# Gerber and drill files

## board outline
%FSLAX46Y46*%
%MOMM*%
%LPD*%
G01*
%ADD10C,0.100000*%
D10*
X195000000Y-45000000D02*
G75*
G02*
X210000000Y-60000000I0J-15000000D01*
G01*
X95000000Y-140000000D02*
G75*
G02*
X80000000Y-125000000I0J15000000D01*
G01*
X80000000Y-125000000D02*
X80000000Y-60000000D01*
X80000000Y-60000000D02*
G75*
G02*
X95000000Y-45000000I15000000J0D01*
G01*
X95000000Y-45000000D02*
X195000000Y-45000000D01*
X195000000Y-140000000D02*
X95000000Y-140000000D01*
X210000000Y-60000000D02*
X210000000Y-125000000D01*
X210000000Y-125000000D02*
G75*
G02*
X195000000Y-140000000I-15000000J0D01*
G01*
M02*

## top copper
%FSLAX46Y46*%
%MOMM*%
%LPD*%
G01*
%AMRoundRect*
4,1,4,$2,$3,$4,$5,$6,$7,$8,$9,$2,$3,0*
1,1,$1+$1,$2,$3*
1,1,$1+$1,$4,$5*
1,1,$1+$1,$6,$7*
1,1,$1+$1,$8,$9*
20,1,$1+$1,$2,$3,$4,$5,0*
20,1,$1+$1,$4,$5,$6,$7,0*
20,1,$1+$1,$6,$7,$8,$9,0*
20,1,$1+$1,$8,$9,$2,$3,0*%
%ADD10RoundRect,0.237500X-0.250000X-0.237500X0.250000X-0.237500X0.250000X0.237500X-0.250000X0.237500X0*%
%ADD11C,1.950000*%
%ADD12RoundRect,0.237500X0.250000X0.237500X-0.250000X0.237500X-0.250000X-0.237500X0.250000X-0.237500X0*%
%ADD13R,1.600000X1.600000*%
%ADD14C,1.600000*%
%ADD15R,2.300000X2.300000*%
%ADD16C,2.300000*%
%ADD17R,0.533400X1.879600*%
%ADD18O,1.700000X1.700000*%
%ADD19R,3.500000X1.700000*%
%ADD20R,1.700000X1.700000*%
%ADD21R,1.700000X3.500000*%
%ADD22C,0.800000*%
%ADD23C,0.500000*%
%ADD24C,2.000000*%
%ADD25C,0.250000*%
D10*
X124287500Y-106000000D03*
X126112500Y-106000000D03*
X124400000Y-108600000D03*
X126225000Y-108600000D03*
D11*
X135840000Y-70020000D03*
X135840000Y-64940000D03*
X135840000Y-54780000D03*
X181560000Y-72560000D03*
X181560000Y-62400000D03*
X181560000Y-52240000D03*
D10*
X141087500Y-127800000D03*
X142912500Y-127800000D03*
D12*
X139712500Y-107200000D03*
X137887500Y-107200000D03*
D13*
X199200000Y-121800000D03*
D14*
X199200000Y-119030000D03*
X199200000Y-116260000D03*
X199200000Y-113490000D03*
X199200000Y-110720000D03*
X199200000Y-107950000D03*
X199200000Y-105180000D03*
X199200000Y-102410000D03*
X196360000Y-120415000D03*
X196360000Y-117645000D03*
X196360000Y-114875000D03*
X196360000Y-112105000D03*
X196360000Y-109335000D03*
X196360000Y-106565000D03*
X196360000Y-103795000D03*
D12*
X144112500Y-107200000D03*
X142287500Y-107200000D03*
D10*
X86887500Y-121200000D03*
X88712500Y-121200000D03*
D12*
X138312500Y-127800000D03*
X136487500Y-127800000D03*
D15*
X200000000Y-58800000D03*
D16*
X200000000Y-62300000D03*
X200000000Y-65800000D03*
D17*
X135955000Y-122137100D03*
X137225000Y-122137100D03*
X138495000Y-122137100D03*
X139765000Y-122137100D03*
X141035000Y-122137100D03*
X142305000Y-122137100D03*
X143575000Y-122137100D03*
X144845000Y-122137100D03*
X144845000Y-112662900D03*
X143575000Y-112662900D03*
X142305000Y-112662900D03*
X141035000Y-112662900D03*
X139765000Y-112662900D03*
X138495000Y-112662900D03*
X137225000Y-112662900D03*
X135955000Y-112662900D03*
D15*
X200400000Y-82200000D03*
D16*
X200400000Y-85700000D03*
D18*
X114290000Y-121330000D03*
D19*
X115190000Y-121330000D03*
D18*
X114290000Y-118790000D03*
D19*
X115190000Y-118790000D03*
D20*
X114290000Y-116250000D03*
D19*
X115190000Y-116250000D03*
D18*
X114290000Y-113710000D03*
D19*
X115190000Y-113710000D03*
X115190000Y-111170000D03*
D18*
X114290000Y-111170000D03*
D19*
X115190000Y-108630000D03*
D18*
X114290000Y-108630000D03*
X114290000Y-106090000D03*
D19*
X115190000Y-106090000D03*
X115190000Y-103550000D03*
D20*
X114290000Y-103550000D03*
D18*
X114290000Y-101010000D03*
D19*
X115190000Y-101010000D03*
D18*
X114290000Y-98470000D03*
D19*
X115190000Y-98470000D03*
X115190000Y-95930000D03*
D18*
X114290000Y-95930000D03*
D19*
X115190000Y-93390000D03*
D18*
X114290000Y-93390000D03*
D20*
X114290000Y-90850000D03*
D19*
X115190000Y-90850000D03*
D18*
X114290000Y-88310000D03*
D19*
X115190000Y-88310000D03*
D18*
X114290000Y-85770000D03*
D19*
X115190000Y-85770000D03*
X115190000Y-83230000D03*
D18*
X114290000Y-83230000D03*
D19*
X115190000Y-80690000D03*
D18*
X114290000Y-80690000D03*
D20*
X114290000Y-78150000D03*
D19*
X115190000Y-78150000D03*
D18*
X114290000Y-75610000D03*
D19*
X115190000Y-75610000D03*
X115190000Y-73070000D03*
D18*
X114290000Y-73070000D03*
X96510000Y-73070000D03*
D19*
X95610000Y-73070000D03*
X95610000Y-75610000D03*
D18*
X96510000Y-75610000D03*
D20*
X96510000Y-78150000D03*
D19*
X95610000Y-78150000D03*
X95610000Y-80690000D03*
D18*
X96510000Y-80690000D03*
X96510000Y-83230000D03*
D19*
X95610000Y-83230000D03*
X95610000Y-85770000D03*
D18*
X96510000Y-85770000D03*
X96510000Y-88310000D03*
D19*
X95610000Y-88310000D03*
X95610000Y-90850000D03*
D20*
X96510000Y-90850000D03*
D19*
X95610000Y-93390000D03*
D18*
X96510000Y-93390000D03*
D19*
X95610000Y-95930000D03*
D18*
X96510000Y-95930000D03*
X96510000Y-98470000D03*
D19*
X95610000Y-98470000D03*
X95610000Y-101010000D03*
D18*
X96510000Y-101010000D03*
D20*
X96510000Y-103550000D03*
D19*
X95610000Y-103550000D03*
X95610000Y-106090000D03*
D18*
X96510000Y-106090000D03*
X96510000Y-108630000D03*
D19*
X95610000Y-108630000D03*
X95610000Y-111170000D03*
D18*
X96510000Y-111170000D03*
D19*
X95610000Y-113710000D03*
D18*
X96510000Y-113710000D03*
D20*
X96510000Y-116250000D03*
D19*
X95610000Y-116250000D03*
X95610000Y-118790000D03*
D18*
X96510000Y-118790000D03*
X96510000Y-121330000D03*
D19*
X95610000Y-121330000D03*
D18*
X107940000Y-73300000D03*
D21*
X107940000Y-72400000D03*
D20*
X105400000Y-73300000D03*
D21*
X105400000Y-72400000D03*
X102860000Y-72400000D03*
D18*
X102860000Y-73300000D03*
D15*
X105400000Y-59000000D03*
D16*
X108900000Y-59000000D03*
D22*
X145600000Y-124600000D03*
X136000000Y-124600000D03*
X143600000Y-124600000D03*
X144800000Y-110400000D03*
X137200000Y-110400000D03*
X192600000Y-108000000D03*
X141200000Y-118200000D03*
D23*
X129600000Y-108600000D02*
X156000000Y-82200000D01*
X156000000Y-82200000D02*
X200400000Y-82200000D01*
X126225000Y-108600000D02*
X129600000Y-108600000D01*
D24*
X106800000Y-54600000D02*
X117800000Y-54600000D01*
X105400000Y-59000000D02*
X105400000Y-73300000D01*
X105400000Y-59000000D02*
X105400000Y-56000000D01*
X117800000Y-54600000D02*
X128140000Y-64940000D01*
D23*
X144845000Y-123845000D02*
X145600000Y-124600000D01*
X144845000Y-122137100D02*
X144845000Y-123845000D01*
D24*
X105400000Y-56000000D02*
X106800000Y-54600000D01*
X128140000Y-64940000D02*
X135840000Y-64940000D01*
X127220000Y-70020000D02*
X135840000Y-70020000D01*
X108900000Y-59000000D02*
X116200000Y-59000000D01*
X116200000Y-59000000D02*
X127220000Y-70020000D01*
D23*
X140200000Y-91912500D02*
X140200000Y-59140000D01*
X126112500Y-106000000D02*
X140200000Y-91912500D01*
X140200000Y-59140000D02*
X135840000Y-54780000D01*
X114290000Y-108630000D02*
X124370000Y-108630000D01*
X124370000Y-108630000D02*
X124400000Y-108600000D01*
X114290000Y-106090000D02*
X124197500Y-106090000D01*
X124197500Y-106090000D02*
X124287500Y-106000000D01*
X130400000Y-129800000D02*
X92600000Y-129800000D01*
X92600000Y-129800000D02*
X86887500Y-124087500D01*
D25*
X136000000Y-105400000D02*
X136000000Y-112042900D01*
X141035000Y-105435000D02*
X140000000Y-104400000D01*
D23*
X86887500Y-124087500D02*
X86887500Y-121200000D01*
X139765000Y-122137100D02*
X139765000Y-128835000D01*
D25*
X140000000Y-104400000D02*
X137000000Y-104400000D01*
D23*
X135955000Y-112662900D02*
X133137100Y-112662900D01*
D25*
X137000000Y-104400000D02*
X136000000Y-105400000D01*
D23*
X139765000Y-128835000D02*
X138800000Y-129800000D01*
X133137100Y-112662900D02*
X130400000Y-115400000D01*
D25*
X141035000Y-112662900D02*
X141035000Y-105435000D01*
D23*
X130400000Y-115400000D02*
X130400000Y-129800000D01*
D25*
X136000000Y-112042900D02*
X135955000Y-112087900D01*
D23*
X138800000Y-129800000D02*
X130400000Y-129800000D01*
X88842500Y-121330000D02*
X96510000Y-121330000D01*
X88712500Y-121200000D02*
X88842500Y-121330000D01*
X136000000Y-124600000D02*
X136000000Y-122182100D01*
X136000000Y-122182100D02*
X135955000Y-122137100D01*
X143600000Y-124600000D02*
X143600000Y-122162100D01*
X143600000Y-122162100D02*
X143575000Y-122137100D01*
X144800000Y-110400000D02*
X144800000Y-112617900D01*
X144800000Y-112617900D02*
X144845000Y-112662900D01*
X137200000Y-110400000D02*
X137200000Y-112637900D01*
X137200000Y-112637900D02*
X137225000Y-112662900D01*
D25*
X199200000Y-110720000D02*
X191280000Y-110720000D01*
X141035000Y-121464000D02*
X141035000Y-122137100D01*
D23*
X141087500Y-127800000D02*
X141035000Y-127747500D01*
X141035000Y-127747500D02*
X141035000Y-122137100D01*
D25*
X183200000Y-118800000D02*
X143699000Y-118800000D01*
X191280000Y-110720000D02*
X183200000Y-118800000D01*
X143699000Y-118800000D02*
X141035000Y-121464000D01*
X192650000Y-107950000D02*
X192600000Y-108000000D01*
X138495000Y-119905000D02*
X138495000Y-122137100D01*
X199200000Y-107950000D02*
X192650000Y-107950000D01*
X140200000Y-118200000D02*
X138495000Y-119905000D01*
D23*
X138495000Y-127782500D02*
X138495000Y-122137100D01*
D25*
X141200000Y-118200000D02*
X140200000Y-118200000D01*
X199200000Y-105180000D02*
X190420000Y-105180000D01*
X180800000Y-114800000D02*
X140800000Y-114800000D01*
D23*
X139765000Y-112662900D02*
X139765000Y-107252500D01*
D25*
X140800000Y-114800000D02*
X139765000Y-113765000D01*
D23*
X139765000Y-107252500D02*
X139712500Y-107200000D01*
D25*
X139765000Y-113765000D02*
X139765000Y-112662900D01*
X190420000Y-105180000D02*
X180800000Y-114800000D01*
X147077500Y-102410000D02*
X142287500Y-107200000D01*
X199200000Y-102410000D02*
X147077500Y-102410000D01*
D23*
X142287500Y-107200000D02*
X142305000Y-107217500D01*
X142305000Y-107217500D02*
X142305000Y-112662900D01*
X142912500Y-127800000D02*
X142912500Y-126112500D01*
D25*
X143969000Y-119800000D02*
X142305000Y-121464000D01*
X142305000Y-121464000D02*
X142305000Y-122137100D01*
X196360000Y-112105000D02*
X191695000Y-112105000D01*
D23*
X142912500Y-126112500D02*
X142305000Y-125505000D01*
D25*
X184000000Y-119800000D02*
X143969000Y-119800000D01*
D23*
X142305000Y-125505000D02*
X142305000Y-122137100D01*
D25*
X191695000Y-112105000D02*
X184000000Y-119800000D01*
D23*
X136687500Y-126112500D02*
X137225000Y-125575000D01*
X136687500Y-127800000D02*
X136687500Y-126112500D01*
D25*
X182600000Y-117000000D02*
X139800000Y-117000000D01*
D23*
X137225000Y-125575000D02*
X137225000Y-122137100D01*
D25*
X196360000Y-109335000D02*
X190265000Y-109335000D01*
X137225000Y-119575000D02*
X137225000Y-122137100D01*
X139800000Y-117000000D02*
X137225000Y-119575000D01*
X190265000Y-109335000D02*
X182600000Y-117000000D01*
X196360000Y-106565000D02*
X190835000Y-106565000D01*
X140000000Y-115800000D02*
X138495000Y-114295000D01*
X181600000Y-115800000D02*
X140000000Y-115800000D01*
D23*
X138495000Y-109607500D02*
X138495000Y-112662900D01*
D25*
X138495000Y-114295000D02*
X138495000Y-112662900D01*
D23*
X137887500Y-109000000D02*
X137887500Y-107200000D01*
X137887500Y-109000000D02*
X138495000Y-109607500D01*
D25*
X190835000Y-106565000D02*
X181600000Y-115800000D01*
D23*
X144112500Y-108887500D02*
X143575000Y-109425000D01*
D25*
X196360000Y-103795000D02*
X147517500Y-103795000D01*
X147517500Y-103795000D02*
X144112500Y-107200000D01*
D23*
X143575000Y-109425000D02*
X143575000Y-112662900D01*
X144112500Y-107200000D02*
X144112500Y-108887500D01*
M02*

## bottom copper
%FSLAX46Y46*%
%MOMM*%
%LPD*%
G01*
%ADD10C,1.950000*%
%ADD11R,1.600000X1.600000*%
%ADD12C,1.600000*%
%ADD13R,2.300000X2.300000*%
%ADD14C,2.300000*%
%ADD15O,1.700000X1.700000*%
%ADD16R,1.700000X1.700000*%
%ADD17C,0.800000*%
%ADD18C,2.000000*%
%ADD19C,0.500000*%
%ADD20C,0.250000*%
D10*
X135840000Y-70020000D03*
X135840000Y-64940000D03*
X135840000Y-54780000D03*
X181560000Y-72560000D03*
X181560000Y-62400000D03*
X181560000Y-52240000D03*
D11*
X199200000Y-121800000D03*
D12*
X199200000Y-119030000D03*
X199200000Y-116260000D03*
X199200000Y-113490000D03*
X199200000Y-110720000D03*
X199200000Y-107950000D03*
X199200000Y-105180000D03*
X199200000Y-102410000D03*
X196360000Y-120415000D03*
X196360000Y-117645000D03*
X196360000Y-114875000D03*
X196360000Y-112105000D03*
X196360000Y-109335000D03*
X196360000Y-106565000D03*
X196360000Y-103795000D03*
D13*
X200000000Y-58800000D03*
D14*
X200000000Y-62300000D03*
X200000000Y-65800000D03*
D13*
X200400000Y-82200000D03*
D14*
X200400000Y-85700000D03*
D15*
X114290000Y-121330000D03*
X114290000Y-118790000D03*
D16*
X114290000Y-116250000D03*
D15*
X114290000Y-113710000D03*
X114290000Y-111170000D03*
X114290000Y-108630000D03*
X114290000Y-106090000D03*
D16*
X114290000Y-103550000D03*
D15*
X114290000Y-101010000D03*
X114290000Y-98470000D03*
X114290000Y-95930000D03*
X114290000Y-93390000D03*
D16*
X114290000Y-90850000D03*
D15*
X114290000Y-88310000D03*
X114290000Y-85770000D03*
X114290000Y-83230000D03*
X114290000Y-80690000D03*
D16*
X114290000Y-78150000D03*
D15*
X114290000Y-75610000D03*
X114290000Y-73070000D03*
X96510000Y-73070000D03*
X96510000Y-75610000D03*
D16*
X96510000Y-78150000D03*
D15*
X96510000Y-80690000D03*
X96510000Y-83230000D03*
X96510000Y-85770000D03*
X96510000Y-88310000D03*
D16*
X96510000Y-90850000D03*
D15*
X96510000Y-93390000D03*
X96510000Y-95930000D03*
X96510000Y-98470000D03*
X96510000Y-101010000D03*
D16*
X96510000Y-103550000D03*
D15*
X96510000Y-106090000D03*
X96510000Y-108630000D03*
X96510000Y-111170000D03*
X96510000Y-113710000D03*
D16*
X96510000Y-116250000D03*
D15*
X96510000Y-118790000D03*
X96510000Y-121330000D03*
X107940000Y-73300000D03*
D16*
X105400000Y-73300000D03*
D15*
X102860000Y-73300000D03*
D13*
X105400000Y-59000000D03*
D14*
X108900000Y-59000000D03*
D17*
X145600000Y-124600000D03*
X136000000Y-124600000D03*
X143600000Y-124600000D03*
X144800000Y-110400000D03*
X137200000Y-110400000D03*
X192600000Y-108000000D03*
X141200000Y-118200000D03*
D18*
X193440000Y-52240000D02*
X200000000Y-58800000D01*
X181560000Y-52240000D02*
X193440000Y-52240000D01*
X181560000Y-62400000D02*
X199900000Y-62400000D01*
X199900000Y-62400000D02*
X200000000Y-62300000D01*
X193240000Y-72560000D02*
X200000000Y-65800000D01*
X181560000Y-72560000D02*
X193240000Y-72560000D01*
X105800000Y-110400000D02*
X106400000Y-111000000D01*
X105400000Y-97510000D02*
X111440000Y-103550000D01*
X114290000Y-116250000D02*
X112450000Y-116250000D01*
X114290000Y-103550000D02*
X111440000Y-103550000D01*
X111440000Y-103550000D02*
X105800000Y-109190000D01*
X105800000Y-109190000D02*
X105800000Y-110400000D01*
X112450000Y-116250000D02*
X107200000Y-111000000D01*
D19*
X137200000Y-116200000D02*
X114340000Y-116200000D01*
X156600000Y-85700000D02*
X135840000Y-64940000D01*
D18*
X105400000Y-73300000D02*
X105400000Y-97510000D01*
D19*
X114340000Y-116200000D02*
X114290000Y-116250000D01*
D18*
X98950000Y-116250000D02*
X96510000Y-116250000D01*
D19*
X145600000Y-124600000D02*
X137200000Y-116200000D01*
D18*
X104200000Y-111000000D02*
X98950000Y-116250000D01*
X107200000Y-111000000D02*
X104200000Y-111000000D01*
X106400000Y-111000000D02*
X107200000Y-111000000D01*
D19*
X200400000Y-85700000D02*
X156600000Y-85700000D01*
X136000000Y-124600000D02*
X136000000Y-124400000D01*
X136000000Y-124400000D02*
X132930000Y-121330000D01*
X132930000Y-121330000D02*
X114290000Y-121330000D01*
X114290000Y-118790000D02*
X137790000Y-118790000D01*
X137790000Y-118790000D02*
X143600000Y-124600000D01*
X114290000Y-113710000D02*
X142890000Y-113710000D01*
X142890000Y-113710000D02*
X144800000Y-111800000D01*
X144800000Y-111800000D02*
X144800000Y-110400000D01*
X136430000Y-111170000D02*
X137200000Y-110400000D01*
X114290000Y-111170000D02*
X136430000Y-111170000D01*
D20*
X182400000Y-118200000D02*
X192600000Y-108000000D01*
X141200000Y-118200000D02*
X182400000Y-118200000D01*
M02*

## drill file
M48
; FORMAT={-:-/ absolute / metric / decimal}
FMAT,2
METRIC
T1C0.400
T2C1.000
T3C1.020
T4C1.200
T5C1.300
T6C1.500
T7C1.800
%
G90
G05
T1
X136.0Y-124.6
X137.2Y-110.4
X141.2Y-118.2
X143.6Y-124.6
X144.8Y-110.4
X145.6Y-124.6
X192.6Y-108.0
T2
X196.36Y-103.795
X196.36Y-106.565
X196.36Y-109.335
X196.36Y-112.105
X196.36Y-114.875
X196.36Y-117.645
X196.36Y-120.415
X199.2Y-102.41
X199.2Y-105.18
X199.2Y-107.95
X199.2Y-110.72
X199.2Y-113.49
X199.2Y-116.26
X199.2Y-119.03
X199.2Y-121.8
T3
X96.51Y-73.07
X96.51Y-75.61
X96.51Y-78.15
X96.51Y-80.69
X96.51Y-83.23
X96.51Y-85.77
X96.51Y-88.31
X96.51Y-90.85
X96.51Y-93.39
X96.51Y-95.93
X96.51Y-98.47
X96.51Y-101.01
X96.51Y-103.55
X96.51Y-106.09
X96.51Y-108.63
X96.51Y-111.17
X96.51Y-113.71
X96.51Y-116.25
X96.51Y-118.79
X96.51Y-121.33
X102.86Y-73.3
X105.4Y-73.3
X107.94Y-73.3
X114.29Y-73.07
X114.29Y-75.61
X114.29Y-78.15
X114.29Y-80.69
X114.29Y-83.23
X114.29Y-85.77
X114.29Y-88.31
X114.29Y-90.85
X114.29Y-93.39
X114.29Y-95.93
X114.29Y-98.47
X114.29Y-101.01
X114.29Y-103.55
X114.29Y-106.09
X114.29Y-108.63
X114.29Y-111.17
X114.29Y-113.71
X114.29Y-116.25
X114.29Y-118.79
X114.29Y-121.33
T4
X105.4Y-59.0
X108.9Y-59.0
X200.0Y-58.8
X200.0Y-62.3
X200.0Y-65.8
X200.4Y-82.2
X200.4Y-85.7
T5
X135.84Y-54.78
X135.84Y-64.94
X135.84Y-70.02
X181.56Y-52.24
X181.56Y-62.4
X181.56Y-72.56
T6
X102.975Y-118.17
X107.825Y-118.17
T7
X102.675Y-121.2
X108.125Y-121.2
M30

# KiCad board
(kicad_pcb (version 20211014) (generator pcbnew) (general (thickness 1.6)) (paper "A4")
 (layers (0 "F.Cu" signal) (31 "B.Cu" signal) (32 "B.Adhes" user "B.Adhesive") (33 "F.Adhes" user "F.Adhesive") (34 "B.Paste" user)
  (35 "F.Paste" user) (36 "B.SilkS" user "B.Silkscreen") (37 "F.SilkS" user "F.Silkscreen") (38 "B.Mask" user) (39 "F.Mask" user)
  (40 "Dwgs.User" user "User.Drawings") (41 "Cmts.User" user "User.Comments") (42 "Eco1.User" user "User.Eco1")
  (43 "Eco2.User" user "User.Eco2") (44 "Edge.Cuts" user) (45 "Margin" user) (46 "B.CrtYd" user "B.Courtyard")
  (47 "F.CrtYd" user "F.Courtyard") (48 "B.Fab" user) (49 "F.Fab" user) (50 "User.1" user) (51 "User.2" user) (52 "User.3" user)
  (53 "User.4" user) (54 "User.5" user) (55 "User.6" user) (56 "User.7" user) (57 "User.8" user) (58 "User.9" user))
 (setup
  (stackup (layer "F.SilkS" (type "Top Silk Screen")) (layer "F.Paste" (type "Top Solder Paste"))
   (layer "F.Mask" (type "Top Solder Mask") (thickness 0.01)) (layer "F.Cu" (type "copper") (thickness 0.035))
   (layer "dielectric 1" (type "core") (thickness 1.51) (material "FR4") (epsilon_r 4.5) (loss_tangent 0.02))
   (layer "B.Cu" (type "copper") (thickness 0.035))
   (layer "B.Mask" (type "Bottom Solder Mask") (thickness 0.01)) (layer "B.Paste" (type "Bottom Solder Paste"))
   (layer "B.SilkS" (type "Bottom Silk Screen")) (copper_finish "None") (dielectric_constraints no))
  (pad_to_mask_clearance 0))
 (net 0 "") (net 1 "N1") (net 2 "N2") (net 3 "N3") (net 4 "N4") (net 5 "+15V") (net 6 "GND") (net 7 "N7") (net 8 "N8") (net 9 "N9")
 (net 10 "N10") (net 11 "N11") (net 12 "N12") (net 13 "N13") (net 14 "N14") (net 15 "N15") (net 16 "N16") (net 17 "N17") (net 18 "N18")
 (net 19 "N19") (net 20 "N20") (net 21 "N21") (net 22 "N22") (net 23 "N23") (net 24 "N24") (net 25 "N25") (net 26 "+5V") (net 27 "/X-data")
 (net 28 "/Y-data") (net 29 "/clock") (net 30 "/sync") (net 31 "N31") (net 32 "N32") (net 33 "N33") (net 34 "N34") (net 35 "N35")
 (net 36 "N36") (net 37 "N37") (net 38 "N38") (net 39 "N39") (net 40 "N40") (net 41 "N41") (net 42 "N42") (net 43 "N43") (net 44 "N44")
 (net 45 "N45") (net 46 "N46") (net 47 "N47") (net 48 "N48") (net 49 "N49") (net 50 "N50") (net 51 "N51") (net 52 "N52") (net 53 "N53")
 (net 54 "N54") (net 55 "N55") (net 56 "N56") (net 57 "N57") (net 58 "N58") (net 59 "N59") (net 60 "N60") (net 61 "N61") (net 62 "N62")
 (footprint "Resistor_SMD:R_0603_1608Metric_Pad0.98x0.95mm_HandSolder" (layer "F.Cu") (at 125.2 106)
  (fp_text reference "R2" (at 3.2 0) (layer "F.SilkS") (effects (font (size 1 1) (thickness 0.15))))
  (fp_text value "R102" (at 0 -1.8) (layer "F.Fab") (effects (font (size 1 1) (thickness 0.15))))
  (pad "1" smd roundrect (at -0.9125 0) (size 0.975 0.95) (layers "F.Cu" "F.Paste" "F.Mask") (roundrect_rratio 0.25) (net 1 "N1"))
  (pad "2" smd roundrect (at 0.9125 0) (size 0.975 0.95) (layers "F.Cu" "F.Paste" "F.Mask") (roundrect_rratio 0.25) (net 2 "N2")))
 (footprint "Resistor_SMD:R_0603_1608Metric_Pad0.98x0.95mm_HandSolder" (layer "F.Cu") (at 125.3125 108.6)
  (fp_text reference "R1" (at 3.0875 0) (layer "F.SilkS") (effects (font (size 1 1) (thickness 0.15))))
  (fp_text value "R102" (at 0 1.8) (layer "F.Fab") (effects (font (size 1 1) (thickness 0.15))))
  (pad "1" smd roundrect (at -0.9125 0) (size 0.975 0.95) (layers "F.Cu" "F.Paste" "F.Mask") (roundrect_rratio 0.25) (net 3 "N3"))
  (pad "2" smd roundrect (at 0.9125 0) (size 0.975 0.95) (layers "F.Cu" "F.Paste" "F.Mask") (roundrect_rratio 0.25) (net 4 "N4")))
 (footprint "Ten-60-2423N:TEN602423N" (layer "F.Cu") (at 135.84 70.2)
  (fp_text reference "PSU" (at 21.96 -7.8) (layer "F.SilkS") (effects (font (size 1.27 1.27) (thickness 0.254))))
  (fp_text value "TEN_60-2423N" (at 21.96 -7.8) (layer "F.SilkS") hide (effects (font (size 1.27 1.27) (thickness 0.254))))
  (pad "1" thru_hole circle locked (at 0 -0.18) (size 1.95 1.95) (drill 1.3) (layers *.Cu *.Mask) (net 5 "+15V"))
  (pad "2" thru_hole circle locked (at 0 -5.26) (size 1.95 1.95) (drill 1.3) (layers *.Cu *.Mask) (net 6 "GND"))
  (pad "3" thru_hole circle locked (at 0 -15.42) (size 1.95 1.95) (drill 1.3) (layers *.Cu *.Mask) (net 2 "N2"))
  (pad "4" thru_hole circle locked (at 45.72 2.36) (size 1.95 1.95) (drill 1.3) (layers *.Cu *.Mask) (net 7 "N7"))
  (pad "5" thru_hole circle locked (at 45.72 -7.8) (size 1.95 1.95) (drill 1.3) (layers *.Cu *.Mask) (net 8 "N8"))
  (pad "6" thru_hole circle locked (at 45.72 -17.96) (size 1.95 1.95) (drill 1.3) (layers *.Cu *.Mask) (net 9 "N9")))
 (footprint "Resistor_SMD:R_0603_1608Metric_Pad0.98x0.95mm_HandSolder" (layer "F.Cu") (at 142 127.8)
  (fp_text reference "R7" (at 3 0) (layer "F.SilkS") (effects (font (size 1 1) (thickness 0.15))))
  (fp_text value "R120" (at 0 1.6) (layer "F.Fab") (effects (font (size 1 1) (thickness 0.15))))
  (pad "1" smd roundrect (at -0.9125 0) (size 0.975 0.95) (layers "F.Cu" "F.Paste" "F.Mask") (roundrect_rratio 0.25) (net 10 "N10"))
  (pad "2" smd roundrect (at 0.9125 0) (size 0.975 0.95) (layers "F.Cu" "F.Paste" "F.Mask") (roundrect_rratio 0.25) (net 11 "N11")))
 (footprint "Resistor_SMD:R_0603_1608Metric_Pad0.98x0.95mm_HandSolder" (layer "F.Cu") (at 138.8 107.2 180)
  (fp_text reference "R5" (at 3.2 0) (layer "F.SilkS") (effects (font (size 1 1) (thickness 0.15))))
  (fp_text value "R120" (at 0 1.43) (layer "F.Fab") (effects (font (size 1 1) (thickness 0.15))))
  (pad "1" smd roundrect (at -0.9125 0 180) (size 0.975 0.95) (layers "F.Cu" "F.Paste" "F.Mask") (roundrect_rratio 0.25) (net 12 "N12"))
  (pad "2" smd roundrect (at 0.9125 0 180) (size 0.975 0.95) (layers "F.Cu" "F.Paste" "F.Mask") (roundrect_rratio 0.25) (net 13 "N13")))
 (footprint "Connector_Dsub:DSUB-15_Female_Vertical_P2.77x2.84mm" (layer "F.Cu") (at 199.2 121.8 -90)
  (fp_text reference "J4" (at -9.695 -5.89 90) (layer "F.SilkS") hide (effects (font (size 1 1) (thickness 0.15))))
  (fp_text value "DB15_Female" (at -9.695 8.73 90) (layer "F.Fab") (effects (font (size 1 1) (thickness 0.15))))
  (pad "1" thru_hole rect (at 0 0 270) (size 1.6 1.6) (drill 1) (layers *.Cu *.Mask) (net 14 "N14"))
  (pad "2" thru_hole circle (at -2.77 0 270) (size 1.6 1.6) (drill 1) (layers *.Cu *.Mask) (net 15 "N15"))
  (pad "3" thru_hole circle (at -5.54 0 270) (size 1.6 1.6) (drill 1) (layers *.Cu *.Mask) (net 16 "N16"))
  (pad "4" thru_hole circle (at -8.31 0 270) (size 1.6 1.6) (drill 1) (layers *.Cu *.Mask) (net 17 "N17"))
  (pad "5" thru_hole circle (at -11.08 0 270) (size 1.6 1.6) (drill 1) (layers *.Cu *.Mask) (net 10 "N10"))
  (pad "6" thru_hole circle (at -13.85 0 270) (size 1.6 1.6) (drill 1) (layers *.Cu *.Mask) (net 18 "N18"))
  (pad "7" thru_hole circle (at -16.62 0 270) (size 1.6 1.6) (drill 1) (layers *.Cu *.Mask) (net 12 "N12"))
  (pad "8" thru_hole circle (at -19.39 0 270) (size 1.6 1.6) (drill 1) (layers *.Cu *.Mask) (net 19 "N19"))
  (pad "9" thru_hole circle (at -1.385 2.84 270) (size 1.6 1.6) (drill 1) (layers *.Cu *.Mask) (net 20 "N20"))
  (pad "10" thru_hole circle (at -4.155 2.84 270) (size 1.6 1.6) (drill 1) (layers *.Cu *.Mask) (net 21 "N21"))
  (pad "11" thru_hole circle (at -6.925 2.84 270) (size 1.6 1.6) (drill 1) (layers *.Cu *.Mask) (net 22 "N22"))
  (pad "12" thru_hole circle (at -9.695 2.84 270) (size 1.6 1.6) (drill 1) (layers *.Cu *.Mask) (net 11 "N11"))
  (pad "13" thru_hole circle (at -12.465 2.84 270) (size 1.6 1.6) (drill 1) (layers *.Cu *.Mask) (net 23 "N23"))
  (pad "14" thru_hole circle (at -15.235 2.84 270) (size 1.6 1.6) (drill 1) (layers *.Cu *.Mask) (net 13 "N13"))
  (pad "15" thru_hole circle (at -18.005 2.84 270) (size 1.6 1.6) (drill 1) (layers *.Cu *.Mask) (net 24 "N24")))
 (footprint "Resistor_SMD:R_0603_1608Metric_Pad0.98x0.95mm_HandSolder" (layer "F.Cu") (at 143.2 107.2 180)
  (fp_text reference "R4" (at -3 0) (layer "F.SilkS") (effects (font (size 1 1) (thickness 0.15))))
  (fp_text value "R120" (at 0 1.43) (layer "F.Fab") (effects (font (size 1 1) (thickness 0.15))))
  (pad "1" smd roundrect (at -0.9125 0 180) (size 0.975 0.95) (layers "F.Cu" "F.Paste" "F.Mask") (roundrect_rratio 0.25) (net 24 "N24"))
  (pad "2" smd roundrect (at 0.9125 0 180) (size 0.975 0.95) (layers "F.Cu" "F.Paste" "F.Mask") (roundrect_rratio 0.25) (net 19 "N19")))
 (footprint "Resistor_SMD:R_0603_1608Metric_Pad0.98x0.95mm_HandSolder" (layer "F.Cu") (at 87.8 121.2)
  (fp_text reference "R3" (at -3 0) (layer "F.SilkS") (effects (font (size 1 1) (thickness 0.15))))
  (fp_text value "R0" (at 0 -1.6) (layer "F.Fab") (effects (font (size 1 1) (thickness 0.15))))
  (pad "1" smd roundrect (at -0.9125 0) (size 0.975 0.95) (layers "F.Cu" "F.Paste" "F.Mask") (roundrect_rratio 0.25) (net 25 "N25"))
  (pad "2" smd roundrect (at 0.9125 0) (size 0.975 0.95) (layers "F.Cu" "F.Paste" "F.Mask") (roundrect_rratio 0.25) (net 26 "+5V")))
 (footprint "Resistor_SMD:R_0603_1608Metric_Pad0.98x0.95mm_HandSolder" (layer "F.Cu") (at 137.4 127.8 180)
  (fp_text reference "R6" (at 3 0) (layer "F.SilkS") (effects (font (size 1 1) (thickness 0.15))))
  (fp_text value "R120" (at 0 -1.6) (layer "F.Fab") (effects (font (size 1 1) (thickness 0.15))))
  (pad "1" smd roundrect (at -0.9125 0 180) (size 0.975 0.95) (layers "F.Cu" "F.Paste" "F.Mask") (roundrect_rratio 0.25) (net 18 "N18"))
  (pad "2" smd roundrect (at 0.9125 0 180) (size 0.975 0.95) (layers "F.Cu" "F.Paste" "F.Mask") (roundrect_rratio 0.25) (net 23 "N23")))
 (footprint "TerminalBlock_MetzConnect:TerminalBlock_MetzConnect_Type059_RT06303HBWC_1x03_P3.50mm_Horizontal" (layer "F.Cu")
  (at 200 58.8 -90)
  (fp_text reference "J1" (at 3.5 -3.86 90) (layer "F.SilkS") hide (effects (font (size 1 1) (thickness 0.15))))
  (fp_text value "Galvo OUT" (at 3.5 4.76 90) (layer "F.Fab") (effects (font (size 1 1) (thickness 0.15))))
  (pad "1" thru_hole rect (at 0 0 270) (size 2.3 2.3) (drill 1.2) (layers *.Cu *.Mask) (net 9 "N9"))
  (pad "2" thru_hole circle (at 3.5 0 270) (size 2.3 2.3) (drill 1.2) (layers *.Cu *.Mask) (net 8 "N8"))
  (pad "3" thru_hole circle (at 7 0 270) (size 2.3 2.3) (drill 1.2) (layers *.Cu *.Mask) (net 7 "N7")))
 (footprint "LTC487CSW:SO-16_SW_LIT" (layer "F.Cu") (at 140.4 117.4 90)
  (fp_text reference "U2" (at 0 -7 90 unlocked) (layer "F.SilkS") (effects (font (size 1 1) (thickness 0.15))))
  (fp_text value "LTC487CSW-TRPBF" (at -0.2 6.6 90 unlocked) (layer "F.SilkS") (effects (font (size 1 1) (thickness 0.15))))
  (pad "1" smd rect (at -4.7371 -4.445 90) (size 1.8796 0.5334) (layers "F.Cu" "F.Paste" "F.Mask") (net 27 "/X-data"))
  (pad "2" smd rect (at -4.7371 -3.175 90) (size 1.8796 0.5334) (layers "F.Cu" "F.Paste" "F.Mask") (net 23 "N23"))
  (pad "3" smd rect (at -4.7371 -1.905 90) (size 1.8796 0.5334) (layers "F.Cu" "F.Paste" "F.Mask") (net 18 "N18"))
  (pad "4" smd rect (at -4.7371 -0.635 90) (size 1.8796 0.5334) (layers "F.Cu" "F.Paste" "F.Mask") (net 25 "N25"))
  (pad "5" smd rect (at -4.7371 0.635 90) (size 1.8796 0.5334) (layers "F.Cu" "F.Paste" "F.Mask") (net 10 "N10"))
  (pad "6" smd rect (at -4.7371 1.905 90) (size 1.8796 0.5334) (layers "F.Cu" "F.Paste" "F.Mask") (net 11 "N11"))
  (pad "7" smd rect (at -4.7371 3.175 90) (size 1.8796 0.5334) (layers "F.Cu" "F.Paste" "F.Mask") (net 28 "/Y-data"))
  (pad "8" smd rect (at -4.7371 4.445 90) (size 1.8796 0.5334) (layers "F.Cu" "F.Paste" "F.Mask") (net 6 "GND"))
  (pad "9" smd rect (at 4.7371 4.445 90) (size 1.8796 0.5334) (layers "F.Cu" "F.Paste" "F.Mask") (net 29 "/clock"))
  (pad "10" smd rect (at 4.7371 3.175 90) (size 1.8796 0.5334) (layers "F.Cu" "F.Paste" "F.Mask") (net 24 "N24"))
  (pad "11" smd rect (at 4.7371 1.905 90) (size 1.8796 0.5334) (layers "F.Cu" "F.Paste" "F.Mask") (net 19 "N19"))
  (pad "12" smd rect (at 4.7371 0.635 90) (size 1.8796 0.5334) (layers "F.Cu" "F.Paste" "F.Mask") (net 25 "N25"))
  (pad "13" smd rect (at 4.7371 -0.635 90) (size 1.8796 0.5334) (layers "F.Cu" "F.Paste" "F.Mask") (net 12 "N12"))
  (pad "14" smd rect (at 4.7371 -1.905 90) (size 1.8796 0.5334) (layers "F.Cu" "F.Paste" "F.Mask") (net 13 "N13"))
  (pad "15" smd rect (at 4.7371 -3.175 90) (size 1.8796 0.5334) (layers "F.Cu" "F.Paste" "F.Mask") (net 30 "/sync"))
  (pad "16" smd rect (at 4.7371 -4.445 90) (size 1.8796 0.5334) (layers "F.Cu" "F.Paste" "F.Mask") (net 25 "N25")))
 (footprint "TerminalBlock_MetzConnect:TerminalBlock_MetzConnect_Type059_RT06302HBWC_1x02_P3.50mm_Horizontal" (layer "F.Cu")
  (at 200.4 82.2 -90)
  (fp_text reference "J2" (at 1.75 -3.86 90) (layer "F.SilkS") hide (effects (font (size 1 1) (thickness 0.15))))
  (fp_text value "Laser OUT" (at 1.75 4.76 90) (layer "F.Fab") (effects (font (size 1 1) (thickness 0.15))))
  (pad "1" thru_hole rect (at 0 0 270) (size 2.3 2.3) (drill 1.2) (layers *.Cu *.Mask) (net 4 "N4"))
  (pad "2" thru_hole circle (at 3.5 0 270) (size 2.3 2.3) (drill 1.2) (layers *.Cu *.Mask) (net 6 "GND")))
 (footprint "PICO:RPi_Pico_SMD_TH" (layer "F.Cu") (at 105.4 97.2 180)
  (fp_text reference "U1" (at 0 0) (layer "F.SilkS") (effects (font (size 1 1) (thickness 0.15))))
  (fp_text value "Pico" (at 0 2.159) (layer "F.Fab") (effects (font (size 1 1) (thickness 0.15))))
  (pad "" np_thru_hole oval (at 2.725 -24 180) (size 1.8 1.8) (drill 1.8) (layers *.Cu *.Mask))
  (pad "" np_thru_hole oval (at 2.425 -20.97 180) (size 1.5 1.5) (drill 1.5) (layers *.Cu *.Mask))
  (pad "" np_thru_hole oval (at -2.725 -24 180) (size 1.8 1.8) (drill 1.8) (layers *.Cu *.Mask))
  (pad "" np_thru_hole oval (at -2.425 -20.97 180) (size 1.5 1.5) (drill 1.5) (layers *.Cu *.Mask))
  (pad "1" thru_hole oval (at -8.89 -24.13 180) (size 1.7 1.7) (drill 1.02) (layers *.Cu *.Mask) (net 27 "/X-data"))
  (pad "1" smd rect (at -8.89 -24.13 180) (size 3.5 1.7) (drill (offset -0.9 0)) (layers "F.Cu" "F.Mask") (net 27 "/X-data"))
  (pad "2" thru_hole oval (at -8.89 -21.59 180) (size 1.7 1.7) (drill 1.02) (layers *.Cu *.Mask) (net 28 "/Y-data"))
  (pad "2" smd rect (at -8.89 -21.59 180) (size 3.5 1.7) (drill (offset -0.9 0)) (layers "F.Cu" "F.Mask") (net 28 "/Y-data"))
  (pad "3" thru_hole rect (at -8.89 -19.05 180) (size 1.7 1.7) (drill 1.02) (layers *.Cu *.Mask) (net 6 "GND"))
  (pad "3" smd rect (at -8.89 -19.05 180) (size 3.5 1.7) (drill (offset -0.9 0)) (layers "F.Cu" "F.Mask") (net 6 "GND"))
  (pad "4" thru_hole oval (at -8.89 -16.51 180) (size 1.7 1.7) (drill 1.02) (layers *.Cu *.Mask) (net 29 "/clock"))
  (pad "4" smd rect (at -8.89 -16.51 180) (size 3.5 1.7) (drill (offset -0.9 0)) (layers "F.Cu" "F.Mask") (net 29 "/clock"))
  (pad "5" smd rect (at -8.89 -13.97 180) (size 3.5 1.7) (drill (offset -0.9 0)) (layers "F.Cu" "F.Mask") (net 30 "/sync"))
  (pad "5" thru_hole oval (at -8.89 -13.97 180) (size 1.7 1.7) (drill 1.02) (layers *.Cu *.Mask) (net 30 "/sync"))
  (pad "6" smd rect (at -8.89 -11.43 180) (size 3.5 1.7) (drill (offset -0.9 0)) (layers "F.Cu" "F.Mask") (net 3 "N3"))
  (pad "6" thru_hole oval (at -8.89 -11.43 180) (size 1.7 1.7) (drill 1.02) (layers *.Cu *.Mask) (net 3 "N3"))
  (pad "7" thru_hole oval (at -8.89 -8.89 180) (size 1.7 1.7) (drill 1.02) (layers *.Cu *.Mask) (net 1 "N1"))
  (pad "7" smd rect (at -8.89 -8.89 180) (size 3.5 1.7) (drill (offset -0.9 0)) (layers "F.Cu" "F.Mask") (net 1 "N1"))
  (pad "8" smd rect (at -8.89 -6.35 180) (size 3.5 1.7) (drill (offset -0.9 0)) (layers "F.Cu" "F.Mask") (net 6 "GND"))
  (pad "8" thru_hole rect (at -8.89 -6.35 180) (size 1.7 1.7) (drill 1.02) (layers *.Cu *.Mask) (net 6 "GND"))
  (pad "9" thru_hole oval (at -8.89 -3.81 180) (size 1.7 1.7) (drill 1.02) (layers *.Cu *.Mask) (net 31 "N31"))
  (pad "9" smd rect (at -8.89 -3.81 180) (size 3.5 1.7) (drill (offset -0.9 0)) (layers "F.Cu" "F.Mask") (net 31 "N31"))
  (pad "10" thru_hole oval (at -8.89 -1.27 180) (size 1.7 1.7) (drill 1.02) (layers *.Cu *.Mask) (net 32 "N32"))
  (pad "10" smd rect (at -8.89 -1.27 180) (size 3.5 1.7) (drill (offset -0.9 0)) (layers "F.Cu" "F.Mask") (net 32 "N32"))
  (pad "11" smd rect (at -8.89 1.27 180) (size 3.5 1.7) (drill (offset -0.9 0)) (layers "F.Cu" "F.Mask") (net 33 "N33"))
  (pad "11" thru_hole oval (at -8.89 1.27 180) (size 1.7 1.7) (drill 1.02) (layers *.Cu *.Mask) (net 33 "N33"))
  (pad "12" smd rect (at -8.89 3.81 180) (size 3.5 1.7) (drill (offset -0.9 0)) (layers "F.Cu" "F.Mask") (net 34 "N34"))
  (pad "12" thru_hole oval (at -8.89 3.81 180) (size 1.7 1.7) (drill 1.02) (layers *.Cu *.Mask) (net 34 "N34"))
  (pad "13" thru_hole rect (at -8.89 6.35 180) (size 1.7 1.7) (drill 1.02) (layers *.Cu *.Mask) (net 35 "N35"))
  (pad "13" smd rect (at -8.89 6.35 180) (size 3.5 1.7) (drill (offset -0.9 0)) (layers "F.Cu" "F.Mask") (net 35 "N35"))
  (pad "14" thru_hole oval (at -8.89 8.89 180) (size 1.7 1.7) (drill 1.02) (layers *.Cu *.Mask) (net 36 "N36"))
  (pad "14" smd rect (at -8.89 8.89 180) (size 3.5 1.7) (drill (offset -0.9 0)) (layers "F.Cu" "F.Mask") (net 36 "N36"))
  (pad "15" thru_hole oval (at -8.89 11.43 180) (size 1.7 1.7) (drill 1.02) (layers *.Cu *.Mask) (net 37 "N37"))
  (pad "15" smd rect (at -8.89 11.43 180) (size 3.5 1.7) (drill (offset -0.9 0)) (layers "F.Cu" "F.Mask") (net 37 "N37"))
  (pad "16" smd rect (at -8.89 13.97 180) (size 3.5 1.7) (drill (offset -0.9 0)) (layers "F.Cu" "F.Mask") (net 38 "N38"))
  (pad "16" thru_hole oval (at -8.89 13.97 180) (size 1.7 1.7) (drill 1.02) (layers *.Cu *.Mask) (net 38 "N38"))
  (pad "17" smd rect (at -8.89 16.51 180) (size 3.5 1.7) (drill (offset -0.9 0)) (layers "F.Cu" "F.Mask") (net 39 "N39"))
  (pad "17" thru_hole oval (at -8.89 16.51 180) (size 1.7 1.7) (drill 1.02) (layers *.Cu *.Mask) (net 39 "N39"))
  (pad "18" thru_hole rect (at -8.89 19.05 180) (size 1.7 1.7) (drill 1.02) (layers *.Cu *.Mask) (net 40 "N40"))
  (pad "18" smd rect (at -8.89 19.05 180) (size 3.5 1.7) (drill (offset -0.9 0)) (layers "F.Cu" "F.Mask") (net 40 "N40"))
  (pad "19" thru_hole oval (at -8.89 21.59 180) (size 1.7 1.7) (drill 1.02) (layers *.Cu *.Mask) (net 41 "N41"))
  (pad "19" smd rect (at -8.89 21.59 180) (size 3.5 1.7) (drill (offset -0.9 0)) (layers "F.Cu" "F.Mask") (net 41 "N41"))
  (pad "20" smd rect (at -8.89 24.13 180) (size 3.5 1.7) (drill (offset -0.9 0)) (layers "F.Cu" "F.Mask") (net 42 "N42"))
  (pad "20" thru_hole oval (at -8.89 24.13 180) (size 1.7 1.7) (drill 1.02) (layers *.Cu *.Mask) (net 42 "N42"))
  (pad "21" thru_hole oval (at 8.89 24.13 180) (size 1.7 1.7) (drill 1.02) (layers *.Cu *.Mask) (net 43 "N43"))
  (pad "21" smd rect (at 8.89 24.13 180) (size 3.5 1.7) (drill (offset 0.9 0)) (layers "F.Cu" "F.Mask") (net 43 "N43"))
  (pad "22" smd rect (at 8.89 21.59 180) (size 3.5 1.7) (drill (offset 0.9 0)) (layers "F.Cu" "F.Mask") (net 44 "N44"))
  (pad "22" thru_hole oval (at 8.89 21.59 180) (size 1.7 1.7) (drill 1.02) (layers *.Cu *.Mask) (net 44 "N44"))
  (pad "23" thru_hole rect (at 8.89 19.05 180) (size 1.7 1.7) (drill 1.02) (layers *.Cu *.Mask) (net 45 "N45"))
  (pad "23" smd rect (at 8.89 19.05 180) (size 3.5 1.7) (drill (offset 0.9 0)) (layers "F.Cu" "F.Mask") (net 45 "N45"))
  (pad "24" smd rect (at 8.89 16.51 180) (size 3.5 1.7) (drill (offset 0.9 0)) (layers "F.Cu" "F.Mask") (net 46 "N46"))
  (pad "24" thru_hole oval (at 8.89 16.51 180) (size 1.7 1.7) (drill 1.02) (layers *.Cu *.Mask) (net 46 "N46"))
  (pad "25" thru_hole oval (at 8.89 13.97 180) (size 1.7 1.7) (drill 1.02) (layers *.Cu *.Mask) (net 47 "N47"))
  (pad "25" smd rect (at 8.89 13.97 180) (size 3.5 1.7) (drill (offset 0.9 0)) (layers "F.Cu" "F.Mask") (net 47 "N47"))
  (pad "26" smd rect (at 8.89 11.43 180) (size 3.5 1.7) (drill (offset 0.9 0)) (layers "F.Cu" "F.Mask") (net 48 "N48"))
  (pad "26" thru_hole oval (at 8.89 11.43 180) (size 1.7 1.7) (drill 1.02) (layers *.Cu *.Mask) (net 48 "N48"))
  (pad "27" thru_hole oval (at 8.89 8.89 180) (size 1.7 1.7) (drill 1.02) (layers *.Cu *.Mask) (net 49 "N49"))
  (pad "27" smd rect (at 8.89 8.89 180) (size 3.5 1.7) (drill (offset 0.9 0)) (layers "F.Cu" "F.Mask") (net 49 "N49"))
  (pad "28" smd rect (at 8.89 6.35 180) (size 3.5 1.7) (drill (offset 0.9 0)) (layers "F.Cu" "F.Mask") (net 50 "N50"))
  (pad "28" thru_hole rect (at 8.89 6.35 180) (size 1.7 1.7) (drill 1.02) (layers *.Cu *.Mask) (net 50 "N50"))
  (pad "29" smd rect (at 8.89 3.81 180) (size 3.5 1.7) (drill (offset 0.9 0)) (layers "F.Cu" "F.Mask") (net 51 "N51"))
  (pad "29" thru_hole oval (at 8.89 3.81 180) (size 1.7 1.7) (drill 1.02) (layers *.Cu *.Mask) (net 51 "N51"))
  (pad "30" smd rect (at 8.89 1.27 180) (size 3.5 1.7) (drill (offset 0.9 0)) (layers "F.Cu" "F.Mask") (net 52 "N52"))
  (pad "30" thru_hole oval (at 8.89 1.27 180) (size 1.7 1.7) (drill 1.02) (layers *.Cu *.Mask) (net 52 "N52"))
  (pad "31" thru_hole oval (at 8.89 -1.27 180) (size 1.7 1.7) (drill 1.02) (layers *.Cu *.Mask) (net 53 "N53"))
  (pad "31" smd rect (at 8.89 -1.27 180) (size 3.5 1.7) (drill (offset 0.9 0)) (layers "F.Cu" "F.Mask") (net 53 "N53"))
  (pad "32" smd rect (at 8.89 -3.81 180) (size 3.5 1.7) (drill (offset 0.9 0)) (layers "F.Cu" "F.Mask") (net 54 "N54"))
  (pad "32" thru_hole oval (at 8.89 -3.81 180) (size 1.7 1.7) (drill 1.02) (layers *.Cu *.Mask) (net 54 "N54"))
  (pad "33" thru_hole rect (at 8.89 -6.35 180) (size 1.7 1.7) (drill 1.02) (layers *.Cu *.Mask) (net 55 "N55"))
  (pad "33" smd rect (at 8.89 -6.35 180) (size 3.5 1.7) (drill (offset 0.9 0)) (layers "F.Cu" "F.Mask") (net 55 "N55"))
  (pad "34" smd rect (at 8.89 -8.89 180) (size 3.5 1.7) (drill (offset 0.9 0)) (layers "F.Cu" "F.Mask") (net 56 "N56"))
  (pad "34" thru_hole oval (at 8.89 -8.89 180) (size 1.7 1.7) (drill 1.02) (layers *.Cu *.Mask) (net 56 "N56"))
  (pad "35" thru_hole oval (at 8.89 -11.43 180) (size 1.7 1.7) (drill 1.02) (layers *.Cu *.Mask) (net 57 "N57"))
  (pad "35" smd rect (at 8.89 -11.43 180) (size 3.5 1.7) (drill (offset 0.9 0)) (layers "F.Cu" "F.Mask") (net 57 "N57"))
  (pad "36" smd rect (at 8.89 -13.97 180) (size 3.5 1.7) (drill (offset 0.9 0)) (layers "F.Cu" "F.Mask") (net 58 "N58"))
  (pad "36" thru_hole oval (at 8.89 -13.97 180) (size 1.7 1.7) (drill 1.02) (layers *.Cu *.Mask) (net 58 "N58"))
  (pad "37" smd rect (at 8.89 -16.51 180) (size 3.5 1.7) (drill (offset 0.9 0)) (layers "F.Cu" "F.Mask") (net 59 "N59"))
  (pad "37" thru_hole oval (at 8.89 -16.51 180) (size 1.7 1.7) (drill 1.02) (layers *.Cu *.Mask) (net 59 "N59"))
  (pad "38" thru_hole rect (at 8.89 -19.05 180) (size 1.7 1.7) (drill 1.02) (layers *.Cu *.Mask) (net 6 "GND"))
  (pad "38" smd rect (at 8.89 -19.05 180) (size 3.5 1.7) (drill (offset 0.9 0)) (layers "F.Cu" "F.Mask") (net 6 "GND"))
  (pad "39" smd rect (at 8.89 -21.59 180) (size 3.5 1.7) (drill (offset 0.9 0)) (layers "F.Cu" "F.Mask") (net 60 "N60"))
  (pad "39" thru_hole oval (at 8.89 -21.59 180) (size 1.7 1.7) (drill 1.02) (layers *.Cu *.Mask) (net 60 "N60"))
  (pad "40" thru_hole oval (at 8.89 -24.13 180) (size 1.7 1.7) (drill 1.02) (layers *.Cu *.Mask) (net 26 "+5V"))
  (pad "40" smd rect (at 8.89 -24.13 180) (size 3.5 1.7) (drill (offset 0.9 0)) (layers "F.Cu" "F.Mask") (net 26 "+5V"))
  (pad "41" thru_hole oval (at -2.54 23.9 180) (size 1.7 1.7) (drill 1.02) (layers *.Cu *.Mask) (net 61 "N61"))
  (pad "41" smd rect (at -2.54 23.9 270) (size 3.5 1.7) (drill (offset -0.9 0)) (layers "F.Cu" "F.Mask") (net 61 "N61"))
  (pad "42" thru_hole rect (at 0 23.9 180) (size 1.7 1.7) (drill 1.02) (layers *.Cu *.Mask) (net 6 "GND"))
  (pad "42" smd rect (at 0 23.9 270) (size 3.5 1.7) (drill (offset -0.9 0)) (layers "F.Cu" "F.Mask") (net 6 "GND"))
  (pad "43" smd rect (at 2.54 23.9 270) (size 3.5 1.7) (drill (offset -0.9 0)) (layers "F.Cu" "F.Mask") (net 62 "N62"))
  (pad "43" thru_hole oval (at 2.54 23.9 180) (size 1.7 1.7) (drill 1.02) (layers *.Cu *.Mask) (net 62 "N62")))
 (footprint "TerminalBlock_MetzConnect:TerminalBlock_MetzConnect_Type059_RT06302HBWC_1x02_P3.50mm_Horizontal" (layer "F.Cu") (at 105.4 59)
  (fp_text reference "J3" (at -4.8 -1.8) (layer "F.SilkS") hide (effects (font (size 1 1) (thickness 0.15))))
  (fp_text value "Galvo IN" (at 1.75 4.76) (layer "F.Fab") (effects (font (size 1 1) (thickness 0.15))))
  (pad "1" thru_hole rect (at 0 0) (size 2.3 2.3) (drill 1.2) (layers *.Cu *.Mask) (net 6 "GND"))
  (pad "2" thru_hole circle (at 3.5 0) (size 2.3 2.3) (drill 1.2) (layers *.Cu *.Mask) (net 5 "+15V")))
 (gr_arc (start 195 45) (mid 205.606602 49.393398) (end 210 60) (layer "Edge.Cuts") (width 0.1))
 (gr_arc (start 95 140) (mid 84.393398 135.606602) (end 80 125) (layer "Edge.Cuts") (width 0.1))
 (gr_line (start 80 125) (end 80 60) (layer "Edge.Cuts") (width 0.1))
 (gr_arc (start 80 60) (mid 84.393398 49.393398) (end 95 45) (layer "Edge.Cuts") (width 0.1))
 (gr_line (start 95 45) (end 195 45) (layer "Edge.Cuts") (width 0.1))
 (gr_line (start 195 140) (end 95 140) (layer "Edge.Cuts") (width 0.1))
 (gr_line (start 210 60) (end 210 125) (layer "Edge.Cuts") (width 0.1))
 (gr_arc (start 210 125) (mid 205.606602 135.606602) (end 195 140) (layer "Edge.Cuts") (width 0.1))
 (segment (start 193.44 52.24) (end 200 58.8) (width 2) (layer "B.Cu") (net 9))
 (segment (start 181.56 52.24) (end 193.44 52.24) (width 2) (layer "B.Cu") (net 9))
 (segment (start 181.56 62.4) (end 199.9 62.4) (width 2) (layer "B.Cu") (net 8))
 (segment (start 199.9 62.4) (end 200 62.3) (width 2) (layer "B.Cu") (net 8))
 (segment (start 193.24 72.56) (end 200 65.8) (width 2) (layer "B.Cu") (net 7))
 (segment (start 181.56 72.56) (end 193.24 72.56) (width 2) (layer "B.Cu") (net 7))
 (segment (start 129.6 108.6) (end 156 82.2) (width 0.5) (layer "F.Cu") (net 4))
 (segment (start 156 82.2) (end 200.4 82.2) (width 0.5) (layer "F.Cu") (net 4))
 (segment (start 126.225 108.6) (end 129.6 108.6) (width 0.5) (layer "F.Cu") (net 4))
 (segment (start 106.8 54.6) (end 117.8 54.6) (width 2) (layer "F.Cu") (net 6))
 (segment (start 105.4 59) (end 105.4 73.3) (width 2) (layer "F.Cu") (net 6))
 (segment (start 105.4 59) (end 105.4 56) (width 2) (layer "F.Cu") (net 6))
 (segment (start 117.8 54.6) (end 128.14 64.94) (width 2) (layer "F.Cu") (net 6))
 (segment (start 144.845 123.845) (end 145.6 124.6) (width 0.5) (layer "F.Cu") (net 6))
 (segment (start 144.845 122.1371) (end 144.845 123.845) (width 0.5) (layer "F.Cu") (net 6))
 (segment (start 105.4 56) (end 106.8 54.6) (width 2) (layer "F.Cu") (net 6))
 (segment (start 128.14 64.94) (end 135.84 64.94) (width 2) (layer "F.Cu") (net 6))
 (via (at 145.6 124.6) (size 0.8) (drill 0.4) (layers "F.Cu" "B.Cu") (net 6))
 (segment (start 105.8 110.4) (end 106.4 111) (width 2) (layer "B.Cu") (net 6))
 (segment (start 105.4 97.51) (end 111.44 103.55) (width 2) (layer "B.Cu") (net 6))
 (segment (start 114.29 116.25) (end 112.45 116.25) (width 2) (layer "B.Cu") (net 6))
 (segment (start 114.29 103.55) (end 111.44 103.55) (width 2) (layer "B.Cu") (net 6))
 (segment (start 111.44 103.55) (end 105.8 109.19) (width 2) (layer "B.Cu") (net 6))
 (segment (start 105.8 109.19) (end 105.8 110.4) (width 2) (layer "B.Cu") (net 6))
 (segment (start 112.45 116.25) (end 107.2 111) (width 2) (layer "B.Cu") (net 6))
 (segment (start 137.2 116.2) (end 114.34 116.2) (width 0.5) (layer "B.Cu") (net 6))
 (segment (start 156.6 85.7) (end 135.84 64.94) (width 0.5) (layer "B.Cu") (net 6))
 (segment (start 105.4 73.3) (end 105.4 97.51) (width 2) (layer "B.Cu") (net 6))
 (segment (start 114.34 116.2) (end 114.29 116.25) (width 0.5) (layer "B.Cu") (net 6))
 (segment (start 98.95 116.25) (end 96.51 116.25) (width 2) (layer "B.Cu") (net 6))
 (segment (start 145.6 124.6) (end 137.2 116.2) (width 0.5) (layer "B.Cu") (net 6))
 (segment (start 104.2 111) (end 98.95 116.25) (width 2) (layer "B.Cu") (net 6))
 (segment (start 107.2 111) (end 104.2 111) (width 2) (layer "B.Cu") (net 6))
 (segment (start 106.4 111) (end 107.2 111) (width 2) (layer "B.Cu") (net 6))
 (segment (start 200.4 85.7) (end 156.6 85.7) (width 0.5) (layer "B.Cu") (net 6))
 (segment (start 127.22 70.02) (end 135.84 70.02) (width 2) (layer "F.Cu") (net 5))
 (segment (start 108.9 59) (end 116.2 59) (width 2) (layer "F.Cu") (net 5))
 (segment (start 116.2 59) (end 127.22 70.02) (width 2) (layer "F.Cu") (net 5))
 (segment (start 140.2 91.9125) (end 140.2 59.14) (width 0.5) (layer "F.Cu") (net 2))
 (segment (start 126.1125 106) (end 140.2 91.9125) (width 0.5) (layer "F.Cu") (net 2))
 (segment (start 140.2 59.14) (end 135.84 54.78) (width 0.5) (layer "F.Cu") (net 2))
 (segment (start 114.29 108.63) (end 124.37 108.63) (width 0.5) (layer "F.Cu") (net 3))
 (segment (start 124.37 108.63) (end 124.4 108.6) (width 0.5) (layer "F.Cu") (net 3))
 (segment (start 114.29 106.09) (end 124.1975 106.09) (width 0.5) (layer "F.Cu") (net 1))
 (segment (start 124.1975 106.09) (end 124.2875 106) (width 0.5) (layer "F.Cu") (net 1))
 (segment (start 130.4 129.8) (end 92.6 129.8) (width 0.5) (layer "F.Cu") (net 25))
 (segment (start 92.6 129.8) (end 86.8875 124.0875) (width 0.5) (layer "F.Cu") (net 25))
 (segment (start 136 105.4) (end 136 112.0429) (width 0.25) (layer "F.Cu") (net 25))
 (segment (start 141.035 105.435) (end 140 104.4) (width 0.25) (layer "F.Cu") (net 25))
 (segment (start 86.8875 124.0875) (end 86.8875 121.2) (width 0.5) (layer "F.Cu") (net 25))
 (segment (start 139.765 122.1371) (end 139.765 128.835) (width 0.5) (layer "F.Cu") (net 25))
 (segment (start 140 104.4) (end 137 104.4) (width 0.25) (layer "F.Cu") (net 25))
 (segment (start 135.955 112.6629) (end 133.1371 112.6629) (width 0.5) (layer "F.Cu") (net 25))
 (segment (start 137 104.4) (end 136 105.4) (width 0.25) (layer "F.Cu") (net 25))
 (segment (start 139.765 128.835) (end 138.8 129.8) (width 0.5) (layer "F.Cu") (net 25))
 (segment (start 133.1371 112.6629) (end 130.4 115.4) (width 0.5) (layer "F.Cu") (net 25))
 (segment (start 141.035 112.6629) (end 141.035 105.435) (width 0.25) (layer "F.Cu") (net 25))
 (segment (start 130.4 115.4) (end 130.4 129.8) (width 0.5) (layer "F.Cu") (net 25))
 (segment (start 136 112.0429) (end 135.955 112.0879) (width 0.25) (layer "F.Cu") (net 25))
 (segment (start 138.8 129.8) (end 130.4 129.8) (width 0.5) (layer "F.Cu") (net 25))
 (segment (start 88.8425 121.33) (end 96.51 121.33) (width 0.5) (layer "F.Cu") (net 26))
 (segment (start 88.7125 121.2) (end 88.8425 121.33) (width 0.5) (layer "F.Cu") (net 26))
 (segment (start 136 124.6) (end 136 122.1821) (width 0.5) (layer "F.Cu") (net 27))
 (segment (start 136 122.1821) (end 135.955 122.1371) (width 0.5) (layer "F.Cu") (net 27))
 (via (at 136 124.6) (size 0.8) (drill 0.4) (layers "F.Cu" "B.Cu") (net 27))
 (segment (start 136 124.6) (end 136 124.4) (width 0.5) (layer "B.Cu") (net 27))
 (segment (start 136 124.4) (end 132.93 121.33) (width 0.5) (layer "B.Cu") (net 27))
 (segment (start 132.93 121.33) (end 114.29 121.33) (width 0.5) (layer "B.Cu") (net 27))
 (segment (start 143.6 124.6) (end 143.6 122.1621) (width 0.5) (layer "F.Cu") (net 28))
 (segment (start 143.6 122.1621) (end 143.575 122.1371) (width 0.5) (layer "F.Cu") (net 28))
 (via (at 143.6 124.6) (size 0.8) (drill 0.4) (layers "F.Cu" "B.Cu") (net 28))
 (segment (start 114.29 118.79) (end 137.79 118.79) (width 0.5) (layer "B.Cu") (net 28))
 (segment (start 137.79 118.79) (end 143.6 124.6) (width 0.5) (layer "B.Cu") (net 28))
 (segment (start 144.8 110.4) (end 144.8 112.6179) (width 0.5) (layer "F.Cu") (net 29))
 (segment (start 144.8 112.6179) (end 144.845 112.6629) (width 0.5) (layer "F.Cu") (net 29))
 (via (at 144.8 110.4) (size 0.8) (drill 0.4) (layers "F.Cu" "B.Cu") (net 29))
 (segment (start 114.29 113.71) (end 142.89 113.71) (width 0.5) (layer "B.Cu") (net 29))
 (segment (start 142.89 113.71) (end 144.8 111.8) (width 0.5) (layer "B.Cu") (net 29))
 (segment (start 144.8 111.8) (end 144.8 110.4) (width 0.5) (layer "B.Cu") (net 29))
 (segment (start 137.2 110.4) (end 137.2 112.6379) (width 0.5) (layer "F.Cu") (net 30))
 (segment (start 137.2 112.6379) (end 137.225 112.6629) (width 0.5) (layer "F.Cu") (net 30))
 (via (at 137.2 110.4) (size 0.8) (drill 0.4) (layers "F.Cu" "B.Cu") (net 30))
 (segment (start 136.43 111.17) (end 137.2 110.4) (width 0.5) (layer "B.Cu") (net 30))
 (segment (start 114.29 111.17) (end 136.43 111.17) (width 0.5) (layer "B.Cu") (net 30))
 (segment (start 199.2 110.72) (end 191.28 110.72) (width 0.25) (layer "F.Cu") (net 10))
 (segment (start 141.035 121.464) (end 141.035 122.1371) (width 0.25) (layer "F.Cu") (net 10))
 (segment (start 141.0875 127.8) (end 141.035 127.7475) (width 0.5) (layer "F.Cu") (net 10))
 (segment (start 141.035 127.7475) (end 141.035 122.1371) (width 0.5) (layer "F.Cu") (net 10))
 (segment (start 183.2 118.8) (end 143.699 118.8) (width 0.25) (layer "F.Cu") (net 10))
 (segment (start 191.28 110.72) (end 183.2 118.8) (width 0.25) (layer "F.Cu") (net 10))
 (segment (start 143.699 118.8) (end 141.035 121.464) (width 0.25) (layer "F.Cu") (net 10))
 (segment (start 192.65 107.95) (end 192.6 108) (width 0.25) (layer "F.Cu") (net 18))
 (segment (start 138.495 119.905) (end 138.495 122.1371) (width 0.25) (layer "F.Cu") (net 18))
 (segment (start 199.2 107.95) (end 192.65 107.95) (width 0.25) (layer "F.Cu") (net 18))
 (segment (start 140.2 118.2) (end 138.495 119.905) (width 0.25) (layer "F.Cu") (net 18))
 (segment (start 138.495 127.7825) (end 138.495 122.1371) (width 0.5) (layer "F.Cu") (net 18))
 (segment (start 141.2 118.2) (end 140.2 118.2) (width 0.25) (layer "F.Cu") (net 18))
 (via (at 192.6 108) (size 0.8) (drill 0.4) (layers "F.Cu" "B.Cu") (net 18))
 (via (at 141.2 118.2) (size 0.8) (drill 0.4) (layers "F.Cu" "B.Cu") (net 18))
 (segment (start 182.4 118.2) (end 192.6 108) (width 0.25) (layer "B.Cu") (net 18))
 (segment (start 141.2 118.2) (end 182.4 118.2) (width 0.25) (layer "B.Cu") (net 18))
 (segment (start 199.2 105.18) (end 190.42 105.18) (width 0.25) (layer "F.Cu") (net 12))
 (segment (start 180.8 114.8) (end 140.8 114.8) (width 0.25) (layer "F.Cu") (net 12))
 (segment (start 139.765 112.6629) (end 139.765 107.2525) (width 0.5) (layer "F.Cu") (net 12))
 (segment (start 140.8 114.8) (end 139.765 113.765) (width 0.25) (layer "F.Cu") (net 12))
 (segment (start 139.765 107.2525) (end 139.7125 107.2) (width 0.5) (layer "F.Cu") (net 12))
 (segment (start 139.765 113.765) (end 139.765 112.6629) (width 0.25) (layer "F.Cu") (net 12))
 (segment (start 190.42 105.18) (end 180.8 114.8) (width 0.25) (layer "F.Cu") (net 12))
 (segment (start 147.0775 102.41) (end 142.2875 107.2) (width 0.25) (layer "F.Cu") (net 19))
 (segment (start 199.2 102.41) (end 147.0775 102.41) (width 0.25) (layer "F.Cu") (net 19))
 (segment (start 142.2875 107.2) (end 142.305 107.2175) (width 0.5) (layer "F.Cu") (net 19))
 (segment (start 142.305 107.2175) (end 142.305 112.6629) (width 0.5) (layer "F.Cu") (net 19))
 (segment (start 142.9125 127.8) (end 142.9125 126.1125) (width 0.5) (layer "F.Cu") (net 11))
 (segment (start 143.969 119.8) (end 142.305 121.464) (width 0.25) (layer "F.Cu") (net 11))
 (segment (start 142.305 121.464) (end 142.305 122.1371) (width 0.25) (layer "F.Cu") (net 11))
 (segment (start 196.36 112.105) (end 191.695 112.105) (width 0.25) (layer "F.Cu") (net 11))
 (segment (start 142.9125 126.1125) (end 142.305 125.505) (width 0.5) (layer "F.Cu") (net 11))
 (segment (start 184 119.8) (end 143.969 119.8) (width 0.25) (layer "F.Cu") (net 11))
 (segment (start 142.305 125.505) (end 142.305 122.1371) (width 0.5) (layer "F.Cu") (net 11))
 (segment (start 191.695 112.105) (end 184 119.8) (width 0.25) (layer "F.Cu") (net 11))
 (segment (start 136.6875 126.1125) (end 137.225 125.575) (width 0.5) (layer "F.Cu") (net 23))
 (segment (start 136.6875 127.8) (end 136.6875 126.1125) (width 0.5) (layer "F.Cu") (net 23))
 (segment (start 182.6 117) (end 139.8 117) (width 0.25) (layer "F.Cu") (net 23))
 (segment (start 137.225 125.575) (end 137.225 122.1371) (width 0.5) (layer "F.Cu") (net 23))
 (segment (start 196.36 109.335) (end 190.265 109.335) (width 0.25) (layer "F.Cu") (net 23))
 (segment (start 137.225 119.575) (end 137.225 122.1371) (width 0.25) (layer "F.Cu") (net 23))
 (segment (start 139.8 117) (end 137.225 119.575) (width 0.25) (layer "F.Cu") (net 23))
 (segment (start 190.265 109.335) (end 182.6 117) (width 0.25) (layer "F.Cu") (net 23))
 (segment (start 196.36 106.565) (end 190.835 106.565) (width 0.25) (layer "F.Cu") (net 13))
 (segment (start 140 115.8) (end 138.495 114.295) (width 0.25) (layer "F.Cu") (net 13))
 (segment (start 181.6 115.8) (end 140 115.8) (width 0.25) (layer "F.Cu") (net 13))
 (segment (start 138.495 109.6075) (end 138.495 112.6629) (width 0.5) (layer "F.Cu") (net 13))
 (segment (start 138.495 114.295) (end 138.495 112.6629) (width 0.25) (layer "F.Cu") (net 13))
 (segment (start 137.8875 109) (end 137.8875 107.2) (width 0.5) (layer "F.Cu") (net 13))
 (segment (start 137.8875 109) (end 138.495 109.6075) (width 0.5) (layer "F.Cu") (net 13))
 (segment (start 190.835 106.565) (end 181.6 115.8) (width 0.25) (layer "F.Cu") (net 13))
 (segment (start 144.1125 108.8875) (end 143.575 109.425) (width 0.5) (layer "F.Cu") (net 24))
 (segment (start 196.36 103.795) (end 147.5175 103.795) (width 0.25) (layer "F.Cu") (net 24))
 (segment (start 147.5175 103.795) (end 144.1125 107.2) (width 0.25) (layer "F.Cu") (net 24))
 (segment (start 143.575 109.425) (end 143.575 112.6629) (width 0.5) (layer "F.Cu") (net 24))
 (segment (start 144.1125 107.2) (end 144.1125 108.8875) (width 0.5) (layer "F.Cu") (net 24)))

